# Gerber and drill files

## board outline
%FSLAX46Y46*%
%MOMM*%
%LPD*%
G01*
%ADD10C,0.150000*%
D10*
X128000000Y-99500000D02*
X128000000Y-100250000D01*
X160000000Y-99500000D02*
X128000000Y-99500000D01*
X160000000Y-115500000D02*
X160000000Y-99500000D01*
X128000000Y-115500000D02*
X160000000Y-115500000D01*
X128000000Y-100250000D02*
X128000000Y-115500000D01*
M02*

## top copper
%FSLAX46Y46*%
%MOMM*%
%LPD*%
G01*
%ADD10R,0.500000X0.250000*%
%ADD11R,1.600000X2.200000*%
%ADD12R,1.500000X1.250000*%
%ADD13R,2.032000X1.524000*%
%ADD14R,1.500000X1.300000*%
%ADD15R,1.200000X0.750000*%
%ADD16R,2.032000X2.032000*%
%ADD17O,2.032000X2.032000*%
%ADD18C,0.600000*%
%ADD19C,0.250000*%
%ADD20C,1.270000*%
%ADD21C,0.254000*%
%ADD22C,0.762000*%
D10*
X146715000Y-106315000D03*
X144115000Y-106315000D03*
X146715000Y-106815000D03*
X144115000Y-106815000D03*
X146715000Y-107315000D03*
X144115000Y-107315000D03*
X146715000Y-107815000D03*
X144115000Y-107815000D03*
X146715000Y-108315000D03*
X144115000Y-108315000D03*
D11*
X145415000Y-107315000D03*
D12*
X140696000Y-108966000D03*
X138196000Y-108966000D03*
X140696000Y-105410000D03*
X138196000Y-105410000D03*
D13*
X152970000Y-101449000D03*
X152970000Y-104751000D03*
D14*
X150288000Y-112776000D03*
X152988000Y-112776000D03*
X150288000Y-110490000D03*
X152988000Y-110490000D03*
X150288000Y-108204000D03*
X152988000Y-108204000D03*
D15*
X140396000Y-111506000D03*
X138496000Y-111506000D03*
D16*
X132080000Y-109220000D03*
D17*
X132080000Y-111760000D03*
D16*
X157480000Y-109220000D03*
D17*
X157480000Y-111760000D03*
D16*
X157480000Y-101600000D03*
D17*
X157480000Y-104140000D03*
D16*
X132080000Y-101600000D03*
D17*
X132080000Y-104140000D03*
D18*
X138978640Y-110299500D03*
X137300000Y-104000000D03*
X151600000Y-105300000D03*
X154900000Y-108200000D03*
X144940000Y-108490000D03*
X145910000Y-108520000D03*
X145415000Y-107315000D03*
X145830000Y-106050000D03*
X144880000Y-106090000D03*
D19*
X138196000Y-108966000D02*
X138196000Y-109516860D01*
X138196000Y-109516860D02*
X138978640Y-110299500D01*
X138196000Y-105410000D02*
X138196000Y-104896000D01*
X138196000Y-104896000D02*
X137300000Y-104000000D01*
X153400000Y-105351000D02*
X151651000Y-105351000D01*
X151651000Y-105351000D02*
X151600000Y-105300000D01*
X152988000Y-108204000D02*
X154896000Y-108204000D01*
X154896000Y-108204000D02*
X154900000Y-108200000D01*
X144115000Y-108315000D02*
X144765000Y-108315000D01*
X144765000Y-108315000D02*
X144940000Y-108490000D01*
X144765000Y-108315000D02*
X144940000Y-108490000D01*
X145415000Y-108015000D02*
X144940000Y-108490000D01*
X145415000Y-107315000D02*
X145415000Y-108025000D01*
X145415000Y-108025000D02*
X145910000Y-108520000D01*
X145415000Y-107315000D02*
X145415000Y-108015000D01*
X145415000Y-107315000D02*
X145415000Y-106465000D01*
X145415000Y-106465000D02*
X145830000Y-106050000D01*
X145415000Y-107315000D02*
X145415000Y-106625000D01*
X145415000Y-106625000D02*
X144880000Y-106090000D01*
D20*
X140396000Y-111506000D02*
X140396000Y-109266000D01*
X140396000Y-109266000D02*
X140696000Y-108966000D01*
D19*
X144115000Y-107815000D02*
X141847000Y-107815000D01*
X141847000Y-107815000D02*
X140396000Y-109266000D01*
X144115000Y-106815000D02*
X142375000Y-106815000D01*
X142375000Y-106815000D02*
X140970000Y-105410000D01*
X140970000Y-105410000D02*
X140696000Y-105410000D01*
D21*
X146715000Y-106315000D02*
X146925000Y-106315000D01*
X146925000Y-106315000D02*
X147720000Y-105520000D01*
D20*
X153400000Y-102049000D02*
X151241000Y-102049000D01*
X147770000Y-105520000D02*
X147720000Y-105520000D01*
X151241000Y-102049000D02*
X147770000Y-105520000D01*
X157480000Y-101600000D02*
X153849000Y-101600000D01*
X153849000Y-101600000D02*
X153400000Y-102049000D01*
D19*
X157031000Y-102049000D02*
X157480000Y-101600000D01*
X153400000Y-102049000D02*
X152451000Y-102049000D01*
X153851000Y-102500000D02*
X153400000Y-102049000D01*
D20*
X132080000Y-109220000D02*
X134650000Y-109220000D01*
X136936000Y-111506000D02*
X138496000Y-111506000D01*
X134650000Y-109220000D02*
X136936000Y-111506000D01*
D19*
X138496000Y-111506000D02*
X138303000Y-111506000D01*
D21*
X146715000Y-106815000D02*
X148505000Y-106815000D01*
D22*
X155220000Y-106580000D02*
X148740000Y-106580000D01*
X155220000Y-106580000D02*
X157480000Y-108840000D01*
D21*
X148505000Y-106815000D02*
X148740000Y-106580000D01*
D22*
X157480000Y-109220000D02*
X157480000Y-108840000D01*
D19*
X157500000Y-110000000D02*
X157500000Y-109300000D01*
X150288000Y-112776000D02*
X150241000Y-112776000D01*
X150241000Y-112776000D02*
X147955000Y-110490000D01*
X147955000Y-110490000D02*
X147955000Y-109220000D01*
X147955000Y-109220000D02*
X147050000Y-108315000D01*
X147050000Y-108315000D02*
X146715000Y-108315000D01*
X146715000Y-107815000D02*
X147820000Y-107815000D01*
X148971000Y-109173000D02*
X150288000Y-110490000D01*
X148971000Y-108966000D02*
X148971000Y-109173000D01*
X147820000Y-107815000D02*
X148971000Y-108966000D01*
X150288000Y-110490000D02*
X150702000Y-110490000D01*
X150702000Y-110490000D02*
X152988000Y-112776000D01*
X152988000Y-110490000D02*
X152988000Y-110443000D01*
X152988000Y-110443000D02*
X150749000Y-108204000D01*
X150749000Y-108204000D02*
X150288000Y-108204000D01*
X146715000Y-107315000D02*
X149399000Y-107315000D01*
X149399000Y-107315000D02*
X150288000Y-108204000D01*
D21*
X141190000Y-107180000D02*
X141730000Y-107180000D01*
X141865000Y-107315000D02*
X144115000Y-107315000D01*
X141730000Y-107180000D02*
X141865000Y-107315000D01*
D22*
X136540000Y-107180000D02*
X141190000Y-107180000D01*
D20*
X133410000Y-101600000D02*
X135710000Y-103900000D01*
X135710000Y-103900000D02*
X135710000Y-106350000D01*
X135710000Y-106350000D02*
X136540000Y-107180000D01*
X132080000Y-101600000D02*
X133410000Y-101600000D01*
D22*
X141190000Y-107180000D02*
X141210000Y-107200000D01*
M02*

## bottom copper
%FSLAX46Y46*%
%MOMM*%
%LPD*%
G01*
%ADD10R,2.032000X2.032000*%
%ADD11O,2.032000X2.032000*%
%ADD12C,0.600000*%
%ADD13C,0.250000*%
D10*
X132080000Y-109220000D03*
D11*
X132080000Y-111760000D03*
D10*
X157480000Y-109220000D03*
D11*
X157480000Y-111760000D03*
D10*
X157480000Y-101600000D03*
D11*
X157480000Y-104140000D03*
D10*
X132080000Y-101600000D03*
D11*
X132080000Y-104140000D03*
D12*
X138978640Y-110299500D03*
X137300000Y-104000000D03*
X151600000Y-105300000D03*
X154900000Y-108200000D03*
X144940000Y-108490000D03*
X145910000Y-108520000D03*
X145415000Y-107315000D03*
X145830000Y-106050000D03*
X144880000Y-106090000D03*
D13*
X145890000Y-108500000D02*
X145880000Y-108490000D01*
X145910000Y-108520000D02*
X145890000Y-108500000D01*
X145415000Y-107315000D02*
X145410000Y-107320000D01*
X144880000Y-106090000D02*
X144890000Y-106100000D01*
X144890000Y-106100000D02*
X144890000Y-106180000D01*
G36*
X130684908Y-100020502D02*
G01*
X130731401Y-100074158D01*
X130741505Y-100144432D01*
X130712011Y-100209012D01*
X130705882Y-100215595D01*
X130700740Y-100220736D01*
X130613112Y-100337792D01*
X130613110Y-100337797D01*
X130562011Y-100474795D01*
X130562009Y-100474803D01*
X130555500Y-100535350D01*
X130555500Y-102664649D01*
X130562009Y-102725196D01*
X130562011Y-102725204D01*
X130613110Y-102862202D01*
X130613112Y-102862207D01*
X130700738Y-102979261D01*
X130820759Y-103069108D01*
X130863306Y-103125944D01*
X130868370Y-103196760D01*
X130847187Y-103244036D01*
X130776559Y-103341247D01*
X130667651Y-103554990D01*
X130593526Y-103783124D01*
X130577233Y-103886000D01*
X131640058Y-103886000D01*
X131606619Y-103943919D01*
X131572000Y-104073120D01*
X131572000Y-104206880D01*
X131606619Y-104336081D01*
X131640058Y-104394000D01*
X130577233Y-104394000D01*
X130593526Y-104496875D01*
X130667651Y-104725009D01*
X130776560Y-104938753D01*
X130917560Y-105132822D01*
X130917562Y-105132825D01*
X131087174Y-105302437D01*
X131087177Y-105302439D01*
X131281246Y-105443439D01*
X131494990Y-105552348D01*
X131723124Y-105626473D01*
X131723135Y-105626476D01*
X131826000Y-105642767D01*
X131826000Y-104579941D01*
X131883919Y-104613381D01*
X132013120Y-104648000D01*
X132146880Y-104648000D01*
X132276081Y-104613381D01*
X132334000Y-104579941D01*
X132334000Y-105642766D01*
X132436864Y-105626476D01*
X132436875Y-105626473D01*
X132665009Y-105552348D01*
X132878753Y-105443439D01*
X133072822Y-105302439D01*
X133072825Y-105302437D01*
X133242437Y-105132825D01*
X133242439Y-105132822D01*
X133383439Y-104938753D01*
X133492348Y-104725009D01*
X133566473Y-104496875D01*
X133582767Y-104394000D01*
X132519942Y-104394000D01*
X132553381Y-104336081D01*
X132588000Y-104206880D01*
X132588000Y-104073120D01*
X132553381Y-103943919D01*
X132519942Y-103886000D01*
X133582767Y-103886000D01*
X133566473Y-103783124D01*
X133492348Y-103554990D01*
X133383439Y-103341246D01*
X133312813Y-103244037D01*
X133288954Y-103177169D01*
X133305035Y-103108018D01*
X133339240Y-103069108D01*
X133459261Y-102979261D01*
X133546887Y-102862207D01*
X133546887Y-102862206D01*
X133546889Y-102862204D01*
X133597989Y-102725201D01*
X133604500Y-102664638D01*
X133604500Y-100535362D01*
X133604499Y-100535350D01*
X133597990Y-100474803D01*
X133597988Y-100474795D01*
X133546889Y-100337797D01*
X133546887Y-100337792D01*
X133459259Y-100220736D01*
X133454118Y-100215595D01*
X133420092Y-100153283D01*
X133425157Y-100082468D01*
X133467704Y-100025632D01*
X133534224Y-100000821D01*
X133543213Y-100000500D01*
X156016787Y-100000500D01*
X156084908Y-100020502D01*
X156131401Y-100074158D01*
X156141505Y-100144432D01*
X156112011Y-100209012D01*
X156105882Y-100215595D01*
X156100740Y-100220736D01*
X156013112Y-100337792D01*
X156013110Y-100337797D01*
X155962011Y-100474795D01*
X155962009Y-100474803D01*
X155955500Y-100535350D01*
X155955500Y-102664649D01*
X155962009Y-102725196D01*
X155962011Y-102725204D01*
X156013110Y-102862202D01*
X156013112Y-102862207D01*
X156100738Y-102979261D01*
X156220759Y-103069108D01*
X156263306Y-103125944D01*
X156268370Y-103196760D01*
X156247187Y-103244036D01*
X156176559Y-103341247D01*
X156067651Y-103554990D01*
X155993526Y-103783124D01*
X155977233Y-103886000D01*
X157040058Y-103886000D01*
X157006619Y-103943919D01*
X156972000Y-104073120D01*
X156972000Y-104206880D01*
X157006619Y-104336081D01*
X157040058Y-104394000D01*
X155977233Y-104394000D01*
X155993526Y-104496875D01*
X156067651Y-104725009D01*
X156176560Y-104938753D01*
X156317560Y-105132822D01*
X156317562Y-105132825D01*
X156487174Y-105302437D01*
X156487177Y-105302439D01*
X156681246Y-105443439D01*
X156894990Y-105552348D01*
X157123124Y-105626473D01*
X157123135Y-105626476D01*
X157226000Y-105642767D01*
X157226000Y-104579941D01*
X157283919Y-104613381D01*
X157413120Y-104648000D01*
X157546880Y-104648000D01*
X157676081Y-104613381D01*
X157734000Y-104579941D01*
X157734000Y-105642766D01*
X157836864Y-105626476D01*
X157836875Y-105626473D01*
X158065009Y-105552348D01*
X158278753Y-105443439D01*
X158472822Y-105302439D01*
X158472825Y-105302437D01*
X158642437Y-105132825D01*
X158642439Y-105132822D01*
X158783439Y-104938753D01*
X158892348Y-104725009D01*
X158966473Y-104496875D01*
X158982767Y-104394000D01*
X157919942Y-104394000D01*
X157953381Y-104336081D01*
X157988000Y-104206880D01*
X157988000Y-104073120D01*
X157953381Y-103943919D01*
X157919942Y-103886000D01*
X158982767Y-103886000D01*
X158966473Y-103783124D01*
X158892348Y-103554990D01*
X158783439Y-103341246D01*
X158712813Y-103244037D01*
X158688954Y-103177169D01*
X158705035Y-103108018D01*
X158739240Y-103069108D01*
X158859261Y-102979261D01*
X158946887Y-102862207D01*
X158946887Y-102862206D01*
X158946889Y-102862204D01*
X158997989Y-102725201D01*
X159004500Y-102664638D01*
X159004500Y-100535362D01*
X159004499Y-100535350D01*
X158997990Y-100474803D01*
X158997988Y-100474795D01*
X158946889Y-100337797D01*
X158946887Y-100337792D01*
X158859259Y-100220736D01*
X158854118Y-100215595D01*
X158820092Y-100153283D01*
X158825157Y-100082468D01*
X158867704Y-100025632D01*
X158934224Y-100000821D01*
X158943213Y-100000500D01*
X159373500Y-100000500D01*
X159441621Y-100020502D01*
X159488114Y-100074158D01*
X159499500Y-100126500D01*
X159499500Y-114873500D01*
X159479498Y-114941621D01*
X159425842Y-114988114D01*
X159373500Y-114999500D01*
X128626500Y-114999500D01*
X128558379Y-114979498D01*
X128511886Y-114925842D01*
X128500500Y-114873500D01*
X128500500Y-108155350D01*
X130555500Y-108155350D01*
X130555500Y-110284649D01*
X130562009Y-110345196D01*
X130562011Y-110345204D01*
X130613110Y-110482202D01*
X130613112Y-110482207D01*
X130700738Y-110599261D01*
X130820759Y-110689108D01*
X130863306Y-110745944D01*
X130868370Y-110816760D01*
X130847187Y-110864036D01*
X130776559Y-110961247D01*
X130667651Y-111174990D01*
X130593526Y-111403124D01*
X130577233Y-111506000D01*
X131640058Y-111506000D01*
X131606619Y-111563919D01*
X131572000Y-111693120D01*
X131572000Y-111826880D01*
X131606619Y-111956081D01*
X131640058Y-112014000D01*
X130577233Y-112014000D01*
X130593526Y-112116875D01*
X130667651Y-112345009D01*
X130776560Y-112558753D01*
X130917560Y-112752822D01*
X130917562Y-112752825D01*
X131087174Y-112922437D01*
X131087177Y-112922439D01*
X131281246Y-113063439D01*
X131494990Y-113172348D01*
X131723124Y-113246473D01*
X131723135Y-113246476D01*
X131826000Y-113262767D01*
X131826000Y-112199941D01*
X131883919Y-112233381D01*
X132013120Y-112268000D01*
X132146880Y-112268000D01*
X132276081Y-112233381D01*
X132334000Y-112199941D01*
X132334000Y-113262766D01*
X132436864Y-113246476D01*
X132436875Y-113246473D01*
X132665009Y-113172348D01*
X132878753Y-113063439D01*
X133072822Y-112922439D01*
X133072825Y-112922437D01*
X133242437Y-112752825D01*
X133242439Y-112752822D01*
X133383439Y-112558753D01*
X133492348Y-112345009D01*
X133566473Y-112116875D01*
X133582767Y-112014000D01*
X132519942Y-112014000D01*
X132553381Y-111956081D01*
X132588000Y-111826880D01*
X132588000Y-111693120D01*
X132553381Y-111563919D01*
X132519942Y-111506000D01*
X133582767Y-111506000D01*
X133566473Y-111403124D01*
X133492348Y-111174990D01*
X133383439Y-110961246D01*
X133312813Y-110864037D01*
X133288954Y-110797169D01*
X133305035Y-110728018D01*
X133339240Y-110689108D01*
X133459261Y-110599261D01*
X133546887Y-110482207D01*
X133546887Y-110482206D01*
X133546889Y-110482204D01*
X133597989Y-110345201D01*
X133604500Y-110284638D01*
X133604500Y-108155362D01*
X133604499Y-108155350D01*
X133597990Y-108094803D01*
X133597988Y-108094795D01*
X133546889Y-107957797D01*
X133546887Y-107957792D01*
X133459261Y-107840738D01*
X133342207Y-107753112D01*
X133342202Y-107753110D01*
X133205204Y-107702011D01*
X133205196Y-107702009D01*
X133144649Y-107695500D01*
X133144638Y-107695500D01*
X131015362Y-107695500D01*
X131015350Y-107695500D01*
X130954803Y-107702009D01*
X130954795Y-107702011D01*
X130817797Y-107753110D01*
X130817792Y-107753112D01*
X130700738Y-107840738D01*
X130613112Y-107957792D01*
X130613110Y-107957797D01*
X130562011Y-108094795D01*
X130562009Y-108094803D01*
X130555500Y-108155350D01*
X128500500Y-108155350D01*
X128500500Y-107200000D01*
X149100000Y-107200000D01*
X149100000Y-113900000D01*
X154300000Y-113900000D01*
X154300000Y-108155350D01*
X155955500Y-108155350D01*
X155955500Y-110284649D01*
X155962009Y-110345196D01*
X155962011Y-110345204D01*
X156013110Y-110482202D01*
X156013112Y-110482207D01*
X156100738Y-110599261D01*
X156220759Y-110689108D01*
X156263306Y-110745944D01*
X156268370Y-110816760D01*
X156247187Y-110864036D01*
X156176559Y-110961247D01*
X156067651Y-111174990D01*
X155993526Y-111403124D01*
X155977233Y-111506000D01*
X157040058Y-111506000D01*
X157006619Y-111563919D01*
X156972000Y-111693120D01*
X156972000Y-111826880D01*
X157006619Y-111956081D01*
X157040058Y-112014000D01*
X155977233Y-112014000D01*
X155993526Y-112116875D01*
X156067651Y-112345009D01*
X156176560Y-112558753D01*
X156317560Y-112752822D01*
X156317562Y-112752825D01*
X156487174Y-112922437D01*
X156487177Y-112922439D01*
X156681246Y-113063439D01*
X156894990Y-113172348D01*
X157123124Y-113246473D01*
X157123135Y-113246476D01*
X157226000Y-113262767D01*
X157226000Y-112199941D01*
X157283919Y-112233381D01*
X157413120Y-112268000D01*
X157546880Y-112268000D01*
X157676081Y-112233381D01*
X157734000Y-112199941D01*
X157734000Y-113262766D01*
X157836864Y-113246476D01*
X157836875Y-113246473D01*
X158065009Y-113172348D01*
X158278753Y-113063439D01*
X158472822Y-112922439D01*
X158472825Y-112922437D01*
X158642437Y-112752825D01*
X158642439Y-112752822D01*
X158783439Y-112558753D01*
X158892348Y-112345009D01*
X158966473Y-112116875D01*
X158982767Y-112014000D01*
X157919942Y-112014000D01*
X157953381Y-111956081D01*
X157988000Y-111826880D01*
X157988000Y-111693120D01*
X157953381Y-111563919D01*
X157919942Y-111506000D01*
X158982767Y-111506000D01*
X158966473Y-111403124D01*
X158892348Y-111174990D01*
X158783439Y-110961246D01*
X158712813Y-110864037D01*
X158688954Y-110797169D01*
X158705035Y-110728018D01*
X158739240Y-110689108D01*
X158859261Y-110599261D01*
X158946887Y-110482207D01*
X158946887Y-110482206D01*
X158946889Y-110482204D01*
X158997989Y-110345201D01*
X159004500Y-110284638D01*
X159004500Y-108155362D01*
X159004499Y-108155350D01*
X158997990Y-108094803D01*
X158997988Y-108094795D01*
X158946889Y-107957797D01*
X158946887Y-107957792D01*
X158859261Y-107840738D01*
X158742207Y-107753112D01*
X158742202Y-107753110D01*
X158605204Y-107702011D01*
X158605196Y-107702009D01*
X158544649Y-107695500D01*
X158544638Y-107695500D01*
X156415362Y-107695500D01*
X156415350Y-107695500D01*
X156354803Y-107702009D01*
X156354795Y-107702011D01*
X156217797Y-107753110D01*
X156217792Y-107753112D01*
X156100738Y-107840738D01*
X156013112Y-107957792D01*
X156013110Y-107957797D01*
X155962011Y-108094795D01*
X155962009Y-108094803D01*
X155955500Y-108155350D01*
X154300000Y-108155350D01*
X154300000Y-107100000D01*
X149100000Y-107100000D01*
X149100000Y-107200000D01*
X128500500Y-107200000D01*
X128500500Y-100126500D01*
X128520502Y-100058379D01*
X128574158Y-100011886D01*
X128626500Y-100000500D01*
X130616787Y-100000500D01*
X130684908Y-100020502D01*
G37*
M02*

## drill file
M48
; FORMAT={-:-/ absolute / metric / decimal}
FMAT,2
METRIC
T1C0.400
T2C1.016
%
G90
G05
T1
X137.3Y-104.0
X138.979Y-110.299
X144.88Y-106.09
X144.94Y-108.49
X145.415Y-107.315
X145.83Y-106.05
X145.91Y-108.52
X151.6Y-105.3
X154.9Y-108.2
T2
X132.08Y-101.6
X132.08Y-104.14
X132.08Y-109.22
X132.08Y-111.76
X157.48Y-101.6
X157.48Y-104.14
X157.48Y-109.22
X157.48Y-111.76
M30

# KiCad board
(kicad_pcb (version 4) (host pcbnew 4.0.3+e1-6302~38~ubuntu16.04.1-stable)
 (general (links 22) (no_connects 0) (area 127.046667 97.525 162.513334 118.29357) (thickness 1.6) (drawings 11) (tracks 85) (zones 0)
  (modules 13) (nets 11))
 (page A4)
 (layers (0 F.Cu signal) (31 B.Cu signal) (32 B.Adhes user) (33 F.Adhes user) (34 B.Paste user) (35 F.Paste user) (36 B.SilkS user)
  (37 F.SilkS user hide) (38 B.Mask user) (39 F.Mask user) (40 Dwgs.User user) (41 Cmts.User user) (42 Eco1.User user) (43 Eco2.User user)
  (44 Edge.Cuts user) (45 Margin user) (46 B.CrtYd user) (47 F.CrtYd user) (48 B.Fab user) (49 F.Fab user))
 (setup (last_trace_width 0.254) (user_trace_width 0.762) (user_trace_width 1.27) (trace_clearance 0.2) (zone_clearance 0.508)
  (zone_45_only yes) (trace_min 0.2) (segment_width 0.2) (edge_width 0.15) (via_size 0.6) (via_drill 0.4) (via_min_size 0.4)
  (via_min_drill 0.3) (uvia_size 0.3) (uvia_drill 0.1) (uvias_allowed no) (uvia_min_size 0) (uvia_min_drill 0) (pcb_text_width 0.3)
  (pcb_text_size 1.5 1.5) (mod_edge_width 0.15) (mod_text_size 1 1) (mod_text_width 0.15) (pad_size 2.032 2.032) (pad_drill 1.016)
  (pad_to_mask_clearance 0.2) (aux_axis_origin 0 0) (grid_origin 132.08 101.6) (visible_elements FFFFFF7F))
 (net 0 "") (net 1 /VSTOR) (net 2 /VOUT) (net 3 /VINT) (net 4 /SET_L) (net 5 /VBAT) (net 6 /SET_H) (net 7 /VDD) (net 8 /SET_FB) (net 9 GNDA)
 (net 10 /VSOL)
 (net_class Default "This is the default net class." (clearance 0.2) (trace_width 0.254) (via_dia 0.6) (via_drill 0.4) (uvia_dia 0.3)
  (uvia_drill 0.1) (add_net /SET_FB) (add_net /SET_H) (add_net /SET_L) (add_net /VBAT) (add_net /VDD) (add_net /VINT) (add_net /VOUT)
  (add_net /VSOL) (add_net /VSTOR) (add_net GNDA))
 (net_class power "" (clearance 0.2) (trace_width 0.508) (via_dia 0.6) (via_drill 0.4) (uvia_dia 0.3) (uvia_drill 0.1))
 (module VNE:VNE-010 (layer F.Cu) (at 145.415 107.315 270)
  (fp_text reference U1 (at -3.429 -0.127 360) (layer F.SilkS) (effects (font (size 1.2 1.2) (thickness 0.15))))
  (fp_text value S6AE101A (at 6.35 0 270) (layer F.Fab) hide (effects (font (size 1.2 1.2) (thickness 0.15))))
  (pad 10 smd rect (at -1 -1.3 270) (size 0.25 0.5) (layers F.Cu F.Paste F.Mask) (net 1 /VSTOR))
  (pad 1 smd rect (at -1 1.3 270) (size 0.25 0.5) (layers F.Cu F.Paste F.Mask))
  (pad 9 smd rect (at -0.5 -1.3 270) (size 0.25 0.5) (layers F.Cu F.Paste F.Mask) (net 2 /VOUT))
  (pad 2 smd rect (at -0.5 1.3 270) (size 0.25 0.5) (layers F.Cu F.Paste F.Mask) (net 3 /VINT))
  (pad 8 smd rect (at 0 -1.3 270) (size 0.25 0.5) (layers F.Cu F.Paste F.Mask) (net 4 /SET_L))
  (pad 3 smd rect (at 0 1.3 270) (size 0.25 0.5) (layers F.Cu F.Paste F.Mask) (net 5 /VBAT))
  (pad 7 smd rect (at 0.5 -1.3 270) (size 0.25 0.5) (layers F.Cu F.Paste F.Mask) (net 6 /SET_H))
  (pad 4 smd rect (at 0.5 1.3 270) (size 0.25 0.5) (layers F.Cu F.Paste F.Mask) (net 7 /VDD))
  (pad 6 smd rect (at 1 -1.3 270) (size 0.25 0.5) (layers F.Cu F.Paste F.Mask) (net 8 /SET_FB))
  (pad 5 smd rect (at 1 1.3 270) (size 0.25 0.5) (layers F.Cu F.Paste F.Mask) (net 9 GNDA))
  (pad 0 smd rect (at 0 0 270) (size 2.2 1.6) (layers F.Cu F.Paste F.Mask) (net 9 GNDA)))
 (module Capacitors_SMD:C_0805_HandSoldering (layer F.Cu) (at 139.446 108.966 180)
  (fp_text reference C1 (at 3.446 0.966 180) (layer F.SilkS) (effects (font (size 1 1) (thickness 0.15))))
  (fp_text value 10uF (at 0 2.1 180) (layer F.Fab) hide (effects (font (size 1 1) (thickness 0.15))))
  (pad 1 smd rect (at -1.25 0 180) (size 1.5 1.25) (layers F.Cu F.Paste F.Mask) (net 7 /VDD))
  (pad 2 smd rect (at 1.25 0 180) (size 1.5 1.25) (layers F.Cu F.Paste F.Mask) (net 9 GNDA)))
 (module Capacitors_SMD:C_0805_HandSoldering (layer F.Cu) (at 139.446 105.41 180)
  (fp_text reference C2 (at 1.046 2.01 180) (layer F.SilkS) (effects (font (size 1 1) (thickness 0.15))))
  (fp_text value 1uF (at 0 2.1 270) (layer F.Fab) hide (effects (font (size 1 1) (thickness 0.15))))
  (pad 1 smd rect (at -1.25 0 180) (size 1.5 1.25) (layers F.Cu F.Paste F.Mask) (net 3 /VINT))
  (pad 2 smd rect (at 1.25 0 180) (size 1.5 1.25) (layers F.Cu F.Paste F.Mask) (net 9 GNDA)))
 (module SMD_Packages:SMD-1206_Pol (layer F.Cu) (at 152.97 103.1 270)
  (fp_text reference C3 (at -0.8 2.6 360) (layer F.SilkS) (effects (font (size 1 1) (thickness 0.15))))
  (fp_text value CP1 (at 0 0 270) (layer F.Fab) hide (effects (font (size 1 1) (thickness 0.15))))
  (pad 1 smd rect (at -1.651 0 270) (size 1.524 2.032) (layers F.Cu F.Paste F.Mask) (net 1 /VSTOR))
  (pad 2 smd rect (at 1.651 0 270) (size 1.524 2.032) (layers F.Cu F.Paste F.Mask) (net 9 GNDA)))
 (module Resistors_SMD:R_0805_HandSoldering (layer F.Cu) (at 151.638 112.776)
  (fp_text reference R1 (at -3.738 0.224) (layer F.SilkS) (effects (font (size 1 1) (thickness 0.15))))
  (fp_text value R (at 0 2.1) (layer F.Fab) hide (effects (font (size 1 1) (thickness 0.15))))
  (pad 1 smd rect (at -1.35 0) (size 1.5 1.3) (layers F.Cu F.Paste F.Mask) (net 8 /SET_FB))
  (pad 2 smd rect (at 1.35 0) (size 1.5 1.3) (layers F.Cu F.Paste F.Mask) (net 6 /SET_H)))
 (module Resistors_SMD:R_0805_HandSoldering (layer F.Cu) (at 151.638 110.49)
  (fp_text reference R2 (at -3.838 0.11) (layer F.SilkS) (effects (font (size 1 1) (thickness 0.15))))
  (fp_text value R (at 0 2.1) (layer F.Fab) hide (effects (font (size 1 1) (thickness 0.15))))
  (pad 1 smd rect (at -1.35 0) (size 1.5 1.3) (layers F.Cu F.Paste F.Mask) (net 6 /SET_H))
  (pad 2 smd rect (at 1.35 0) (size 1.5 1.3) (layers F.Cu F.Paste F.Mask) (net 4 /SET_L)))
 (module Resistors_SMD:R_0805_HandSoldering (layer F.Cu) (at 151.638 108.204)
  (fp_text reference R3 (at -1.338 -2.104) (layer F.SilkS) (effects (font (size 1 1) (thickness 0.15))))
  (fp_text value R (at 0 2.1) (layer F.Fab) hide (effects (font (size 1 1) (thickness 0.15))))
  (pad 1 smd rect (at -1.35 0) (size 1.5 1.3) (layers F.Cu F.Paste F.Mask) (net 4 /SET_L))
  (pad 2 smd rect (at 1.35 0) (size 1.5 1.3) (layers F.Cu F.Paste F.Mask) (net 9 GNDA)))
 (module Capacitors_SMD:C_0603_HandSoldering (layer F.Cu) (at 139.446 111.506 180)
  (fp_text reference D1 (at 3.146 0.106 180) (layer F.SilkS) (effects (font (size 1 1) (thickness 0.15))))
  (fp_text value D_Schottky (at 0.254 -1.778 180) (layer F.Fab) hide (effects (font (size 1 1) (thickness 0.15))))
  (pad 1 smd rect (at -0.95 0 180) (size 1.2 0.75) (layers F.Cu F.Paste F.Mask) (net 7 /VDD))
  (pad 2 smd rect (at 0.95 0 180) (size 1.2 0.75) (layers F.Cu F.Paste F.Mask) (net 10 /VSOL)))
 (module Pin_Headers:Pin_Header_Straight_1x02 (layer F.Cu) (at 132.08 109.22)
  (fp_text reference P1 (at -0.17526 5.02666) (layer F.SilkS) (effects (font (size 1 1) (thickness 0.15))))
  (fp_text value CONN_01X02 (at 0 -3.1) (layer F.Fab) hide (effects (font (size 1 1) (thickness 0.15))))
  (pad 1 thru_hole rect (at 0 0) (size 2.032 2.032) (drill 1.016) (layers *.Cu *.Mask F.SilkS) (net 10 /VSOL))
  (pad 2 thru_hole oval (at 0 2.54) (size 2.032 2.032) (drill 1.016) (layers *.Cu *.Mask F.SilkS) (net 9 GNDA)))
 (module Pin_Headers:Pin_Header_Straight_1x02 (layer F.Cu) (at 157.48 109.22)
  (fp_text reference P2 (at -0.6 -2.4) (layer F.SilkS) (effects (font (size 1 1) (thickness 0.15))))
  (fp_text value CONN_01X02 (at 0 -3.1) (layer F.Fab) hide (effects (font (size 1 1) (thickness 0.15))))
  (pad 1 thru_hole rect (at 0 0) (size 2.032 2.032) (drill 1.016) (layers *.Cu *.Mask F.SilkS) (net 2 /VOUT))
  (pad 2 thru_hole oval (at 0 2.54) (size 2.032 2.032) (drill 1.016) (layers *.Cu *.Mask F.SilkS) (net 9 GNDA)))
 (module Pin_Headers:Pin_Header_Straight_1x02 (layer F.Cu) (at 157.48 101.6)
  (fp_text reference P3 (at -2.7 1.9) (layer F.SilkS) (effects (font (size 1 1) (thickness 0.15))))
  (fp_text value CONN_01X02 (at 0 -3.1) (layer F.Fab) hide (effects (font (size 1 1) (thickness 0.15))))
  (pad 1 thru_hole rect (at 0 0) (size 2.032 2.032) (drill 1.016) (layers *.Cu *.Mask F.SilkS) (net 1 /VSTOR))
  (pad 2 thru_hole oval (at 0 2.54) (size 2.032 2.032) (drill 1.016) (layers *.Cu *.Mask F.SilkS) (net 9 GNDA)))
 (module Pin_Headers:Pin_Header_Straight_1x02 (layer F.Cu) (at 132.08 101.6)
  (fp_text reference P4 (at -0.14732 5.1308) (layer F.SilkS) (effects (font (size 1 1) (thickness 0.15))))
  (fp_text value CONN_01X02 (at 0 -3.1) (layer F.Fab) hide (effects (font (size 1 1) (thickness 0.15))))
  (pad 1 thru_hole rect (at 0 0) (size 2.032 2.032) (drill 1.016) (layers *.Cu *.Mask F.SilkS) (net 5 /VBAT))
  (pad 2 thru_hole oval (at 0 2.54) (size 2.032 2.032) (drill 1.016) (layers *.Cu *.Mask F.SilkS) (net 9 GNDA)))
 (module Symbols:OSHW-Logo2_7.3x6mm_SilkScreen (layer F.Cu) (at 143.7 112.1)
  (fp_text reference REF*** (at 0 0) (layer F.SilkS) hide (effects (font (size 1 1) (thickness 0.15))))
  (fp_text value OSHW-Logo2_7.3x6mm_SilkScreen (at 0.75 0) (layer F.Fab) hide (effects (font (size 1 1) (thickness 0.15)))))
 (gr_line (start 128 99.5) (end 128 100.25) (angle 90) (layer Edge.Cuts) (width 0.15))
 (gr_line (start 160 99.5) (end 128 99.5) (angle 90) (layer Edge.Cuts) (width 0.15))
 (gr_line (start 160 115.5) (end 160 99.5) (angle 90) (layer Edge.Cuts) (width 0.15))
 (gr_line (start 128 115.5) (end 160 115.5) (angle 90) (layer Edge.Cuts) (width 0.15))
 (gr_line (start 128 100.25) (end 128 115.5) (angle 90) (layer Edge.Cuts) (width 0.15))
 (segment (start 138.196 108.966) (end 138.196 109.51686) (width 0.25) (layer F.Cu) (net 9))
 (segment (start 138.196 109.51686) (end 138.97864 110.2995) (width 0.25) (layer F.Cu) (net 9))
 (via (at 138.97864 110.2995) (size 0.6) (drill 0.4) (layers F.Cu B.Cu) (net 9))
 (segment (start 138.196 105.41) (end 138.196 104.896) (width 0.25) (layer F.Cu) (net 9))
 (segment (start 138.196 104.896) (end 137.3 104) (width 0.25) (layer F.Cu) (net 9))
 (via (at 137.3 104) (size 0.6) (drill 0.4) (layers F.Cu B.Cu) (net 9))
 (segment (start 153.4 105.351) (end 151.651 105.351) (width 0.25) (layer F.Cu) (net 9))
 (via (at 151.6 105.3) (size 0.6) (drill 0.4) (layers F.Cu B.Cu) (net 9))
 (segment (start 151.651 105.351) (end 151.6 105.3) (width 0.25) (layer F.Cu) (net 9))
 (segment (start 152.988 108.204) (end 154.896 108.204) (width 0.25) (layer F.Cu) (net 9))
 (via (at 154.9 108.2) (size 0.6) (drill 0.4) (layers F.Cu B.Cu) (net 9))
 (segment (start 154.896 108.204) (end 154.9 108.2) (width 0.25) (layer F.Cu) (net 9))
 (segment (start 144.115 108.315) (end 144.765 108.315) (width 0.25) (layer F.Cu) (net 9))
 (segment (start 144.765 108.315) (end 144.94 108.49) (width 0.25) (layer F.Cu) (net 9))
 (segment (start 144.765 108.315) (end 144.94 108.49) (width 0.25) (layer F.Cu) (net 9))
 (via (at 144.94 108.49) (size 0.6) (drill 0.4) (layers F.Cu B.Cu) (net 9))
 (segment (start 145.415 108.015) (end 144.94 108.49) (width 0.25) (layer F.Cu) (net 9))
 (segment (start 145.415 107.315) (end 145.415 108.025) (width 0.25) (layer F.Cu) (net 9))
 (segment (start 145.415 108.025) (end 145.91 108.52) (width 0.25) (layer F.Cu) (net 9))
 (segment (start 145.89 108.5) (end 145.88 108.49) (width 0.25) (layer B.Cu) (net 9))
 (segment (start 145.91 108.52) (end 145.89 108.5) (width 0.25) (layer B.Cu) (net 9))
 (via (at 145.91 108.52) (size 0.6) (drill 0.4) (layers F.Cu B.Cu) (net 9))
 (segment (start 145.415 107.315) (end 145.415 108.015) (width 0.25) (layer F.Cu) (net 9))
 (via (at 145.415 107.315) (size 0.6) (drill 0.4) (layers F.Cu B.Cu) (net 9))
 (segment (start 145.415 107.315) (end 145.41 107.32) (width 0.25) (layer B.Cu) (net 9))
 (segment (start 145.415 107.315) (end 145.415 106.465) (width 0.25) (layer F.Cu) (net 9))
 (segment (start 145.415 106.465) (end 145.83 106.05) (width 0.25) (layer F.Cu) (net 9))
 (via (at 145.83 106.05) (size 0.6) (drill 0.4) (layers F.Cu B.Cu) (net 9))
 (segment (start 145.415 107.315) (end 145.415 106.625) (width 0.25) (layer F.Cu) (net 9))
 (segment (start 145.415 106.625) (end 144.88 106.09) (width 0.25) (layer F.Cu) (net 9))
 (via (at 144.88 106.09) (size 0.6) (drill 0.4) (layers F.Cu B.Cu) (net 9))
 (segment (start 144.88 106.09) (end 144.89 106.1) (width 0.25) (layer B.Cu) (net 9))
 (segment (start 144.89 106.1) (end 144.89 106.18) (width 0.25) (layer B.Cu) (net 9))
 (segment (start 140.396 111.506) (end 140.396 109.266) (width 1.27) (layer F.Cu) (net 7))
 (segment (start 140.396 109.266) (end 140.696 108.966) (width 1.27) (layer F.Cu) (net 7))
 (segment (start 144.115 107.815) (end 141.847 107.815) (width 0.25) (layer F.Cu) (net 7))
 (segment (start 141.847 107.815) (end 140.396 109.266) (width 0.25) (layer F.Cu) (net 7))
 (segment (start 144.115 106.815) (end 142.375 106.815) (width 0.25) (layer F.Cu) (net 3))
 (segment (start 142.375 106.815) (end 140.97 105.41) (width 0.25) (layer F.Cu) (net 3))
 (segment (start 140.97 105.41) (end 140.696 105.41) (width 0.25) (layer F.Cu) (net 3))
 (segment (start 146.715 106.315) (end 146.925 106.315) (width 0.254) (layer F.Cu) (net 1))
 (segment (start 146.925 106.315) (end 147.72 105.52) (width 0.254) (layer F.Cu) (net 1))
 (segment (start 153.4 102.049) (end 151.241 102.049) (width 1.27) (layer F.Cu) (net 1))
 (segment (start 147.77 105.52) (end 147.72 105.52) (width 1.27) (layer F.Cu) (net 1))
 (segment (start 151.241 102.049) (end 147.77 105.52) (width 1.27) (layer F.Cu) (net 1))
 (segment (start 157.48 101.6) (end 153.849 101.6) (width 1.27) (layer F.Cu) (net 1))
 (segment (start 153.849 101.6) (end 153.4 102.049) (width 1.27) (layer F.Cu) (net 1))
 (segment (start 157.031 102.049) (end 157.48 101.6) (width 0.25) (layer F.Cu) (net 1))
 (segment (start 153.4 102.049) (end 152.451 102.049) (width 0.25) (layer F.Cu) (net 1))
 (segment (start 153.851 102.5) (end 153.4 102.049) (width 0.25) (layer F.Cu) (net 1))
 (segment (start 132.08 109.22) (end 134.65 109.22) (width 1.27) (layer F.Cu) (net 10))
 (segment (start 136.936 111.506) (end 138.496 111.506) (width 1.27) (layer F.Cu) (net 10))
 (segment (start 134.65 109.22) (end 136.936 111.506) (width 1.27) (layer F.Cu) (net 10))
 (segment (start 138.496 111.506) (end 138.303 111.506) (width 0.25) (layer F.Cu) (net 10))
 (segment (start 146.715 106.815) (end 148.505 106.815) (width 0.254) (layer F.Cu) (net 2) (status 400000))
 (segment (start 155.22 106.58) (end 148.74 106.58) (width 0.762) (layer F.Cu) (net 2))
 (segment (start 155.22 106.58) (end 157.48 108.84) (width 0.762) (layer F.Cu) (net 2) (status 800000))
 (segment (start 148.505 106.815) (end 148.74 106.58) (width 0.254) (layer F.Cu) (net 2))
 (segment (start 157.48 109.22) (end 157.48 108.84) (width 0.762) (layer F.Cu) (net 2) (status C00000))
 (segment (start 157.5 110) (end 157.5 109.3) (width 0.25) (layer F.Cu) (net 2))
 (segment (start 150.288 112.776) (end 150.241 112.776) (width 0.25) (layer F.Cu) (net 8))
 (segment (start 150.241 112.776) (end 147.955 110.49) (width 0.25) (layer F.Cu) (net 8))
 (segment (start 147.955 110.49) (end 147.955 109.22) (width 0.25) (layer F.Cu) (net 8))
 (segment (start 147.955 109.22) (end 147.05 108.315) (width 0.25) (layer F.Cu) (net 8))
 (segment (start 147.05 108.315) (end 146.715 108.315) (width 0.25) (layer F.Cu) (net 8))
 (segment (start 146.715 107.815) (end 147.82 107.815) (width 0.25) (layer F.Cu) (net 6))
 (segment (start 148.971 109.173) (end 150.288 110.49) (width 0.25) (layer F.Cu) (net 6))
 (segment (start 148.971 108.966) (end 148.971 109.173) (width 0.25) (layer F.Cu) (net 6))
 (segment (start 147.82 107.815) (end 148.971 108.966) (width 0.25) (layer F.Cu) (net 6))
 (segment (start 150.288 110.49) (end 150.702 110.49) (width 0.25) (layer F.Cu) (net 6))
 (segment (start 150.702 110.49) (end 152.988 112.776) (width 0.25) (layer F.Cu) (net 6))
 (segment (start 152.988 110.49) (end 152.988 110.443) (width 0.25) (layer F.Cu) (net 4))
 (segment (start 152.988 110.443) (end 150.749 108.204) (width 0.25) (layer F.Cu) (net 4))
 (segment (start 150.749 108.204) (end 150.288 108.204) (width 0.25) (layer F.Cu) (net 4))
 (segment (start 146.715 107.315) (end 149.399 107.315) (width 0.25) (layer F.Cu) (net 4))
 (segment (start 149.399 107.315) (end 150.288 108.204) (width 0.25) (layer F.Cu) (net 4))
 (segment (start 141.19 107.18) (end 141.73 107.18) (width 0.254) (layer F.Cu) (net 5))
 (segment (start 141.865 107.315) (end 144.115 107.315) (width 0.254) (layer F.Cu) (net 5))
 (segment (start 141.73 107.18) (end 141.865 107.315) (width 0.254) (layer F.Cu) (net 5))
 (segment (start 136.54 107.18) (end 141.19 107.18) (width 0.762) (layer F.Cu) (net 5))
 (segment (start 133.41 101.6) (end 135.71 103.9) (width 1.27) (layer F.Cu) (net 5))
 (segment (start 135.71 103.9) (end 135.71 106.35) (width 1.27) (layer F.Cu) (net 5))
 (segment (start 135.71 106.35) (end 136.54 107.18) (width 1.27) (layer F.Cu) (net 5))
 (segment (start 132.08 101.6) (end 133.41 101.6) (width 1.27) (layer F.Cu) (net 5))
 (segment (start 141.19 107.18) (end 141.21 107.2) (width 0.762) (layer F.Cu) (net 5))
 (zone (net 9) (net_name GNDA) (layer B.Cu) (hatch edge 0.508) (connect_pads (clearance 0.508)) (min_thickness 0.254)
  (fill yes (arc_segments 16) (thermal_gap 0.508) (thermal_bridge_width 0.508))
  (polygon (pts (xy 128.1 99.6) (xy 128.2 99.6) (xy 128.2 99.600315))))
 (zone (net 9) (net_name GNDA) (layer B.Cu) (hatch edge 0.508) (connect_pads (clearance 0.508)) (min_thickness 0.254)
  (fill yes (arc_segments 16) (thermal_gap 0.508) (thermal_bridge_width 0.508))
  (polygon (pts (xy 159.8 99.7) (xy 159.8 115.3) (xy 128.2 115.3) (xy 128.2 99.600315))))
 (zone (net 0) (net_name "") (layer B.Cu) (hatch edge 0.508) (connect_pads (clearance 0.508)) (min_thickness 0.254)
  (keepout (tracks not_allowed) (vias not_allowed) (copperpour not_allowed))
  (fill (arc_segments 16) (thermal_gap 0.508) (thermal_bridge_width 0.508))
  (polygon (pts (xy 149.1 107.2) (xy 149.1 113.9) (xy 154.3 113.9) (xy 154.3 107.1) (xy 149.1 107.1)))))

